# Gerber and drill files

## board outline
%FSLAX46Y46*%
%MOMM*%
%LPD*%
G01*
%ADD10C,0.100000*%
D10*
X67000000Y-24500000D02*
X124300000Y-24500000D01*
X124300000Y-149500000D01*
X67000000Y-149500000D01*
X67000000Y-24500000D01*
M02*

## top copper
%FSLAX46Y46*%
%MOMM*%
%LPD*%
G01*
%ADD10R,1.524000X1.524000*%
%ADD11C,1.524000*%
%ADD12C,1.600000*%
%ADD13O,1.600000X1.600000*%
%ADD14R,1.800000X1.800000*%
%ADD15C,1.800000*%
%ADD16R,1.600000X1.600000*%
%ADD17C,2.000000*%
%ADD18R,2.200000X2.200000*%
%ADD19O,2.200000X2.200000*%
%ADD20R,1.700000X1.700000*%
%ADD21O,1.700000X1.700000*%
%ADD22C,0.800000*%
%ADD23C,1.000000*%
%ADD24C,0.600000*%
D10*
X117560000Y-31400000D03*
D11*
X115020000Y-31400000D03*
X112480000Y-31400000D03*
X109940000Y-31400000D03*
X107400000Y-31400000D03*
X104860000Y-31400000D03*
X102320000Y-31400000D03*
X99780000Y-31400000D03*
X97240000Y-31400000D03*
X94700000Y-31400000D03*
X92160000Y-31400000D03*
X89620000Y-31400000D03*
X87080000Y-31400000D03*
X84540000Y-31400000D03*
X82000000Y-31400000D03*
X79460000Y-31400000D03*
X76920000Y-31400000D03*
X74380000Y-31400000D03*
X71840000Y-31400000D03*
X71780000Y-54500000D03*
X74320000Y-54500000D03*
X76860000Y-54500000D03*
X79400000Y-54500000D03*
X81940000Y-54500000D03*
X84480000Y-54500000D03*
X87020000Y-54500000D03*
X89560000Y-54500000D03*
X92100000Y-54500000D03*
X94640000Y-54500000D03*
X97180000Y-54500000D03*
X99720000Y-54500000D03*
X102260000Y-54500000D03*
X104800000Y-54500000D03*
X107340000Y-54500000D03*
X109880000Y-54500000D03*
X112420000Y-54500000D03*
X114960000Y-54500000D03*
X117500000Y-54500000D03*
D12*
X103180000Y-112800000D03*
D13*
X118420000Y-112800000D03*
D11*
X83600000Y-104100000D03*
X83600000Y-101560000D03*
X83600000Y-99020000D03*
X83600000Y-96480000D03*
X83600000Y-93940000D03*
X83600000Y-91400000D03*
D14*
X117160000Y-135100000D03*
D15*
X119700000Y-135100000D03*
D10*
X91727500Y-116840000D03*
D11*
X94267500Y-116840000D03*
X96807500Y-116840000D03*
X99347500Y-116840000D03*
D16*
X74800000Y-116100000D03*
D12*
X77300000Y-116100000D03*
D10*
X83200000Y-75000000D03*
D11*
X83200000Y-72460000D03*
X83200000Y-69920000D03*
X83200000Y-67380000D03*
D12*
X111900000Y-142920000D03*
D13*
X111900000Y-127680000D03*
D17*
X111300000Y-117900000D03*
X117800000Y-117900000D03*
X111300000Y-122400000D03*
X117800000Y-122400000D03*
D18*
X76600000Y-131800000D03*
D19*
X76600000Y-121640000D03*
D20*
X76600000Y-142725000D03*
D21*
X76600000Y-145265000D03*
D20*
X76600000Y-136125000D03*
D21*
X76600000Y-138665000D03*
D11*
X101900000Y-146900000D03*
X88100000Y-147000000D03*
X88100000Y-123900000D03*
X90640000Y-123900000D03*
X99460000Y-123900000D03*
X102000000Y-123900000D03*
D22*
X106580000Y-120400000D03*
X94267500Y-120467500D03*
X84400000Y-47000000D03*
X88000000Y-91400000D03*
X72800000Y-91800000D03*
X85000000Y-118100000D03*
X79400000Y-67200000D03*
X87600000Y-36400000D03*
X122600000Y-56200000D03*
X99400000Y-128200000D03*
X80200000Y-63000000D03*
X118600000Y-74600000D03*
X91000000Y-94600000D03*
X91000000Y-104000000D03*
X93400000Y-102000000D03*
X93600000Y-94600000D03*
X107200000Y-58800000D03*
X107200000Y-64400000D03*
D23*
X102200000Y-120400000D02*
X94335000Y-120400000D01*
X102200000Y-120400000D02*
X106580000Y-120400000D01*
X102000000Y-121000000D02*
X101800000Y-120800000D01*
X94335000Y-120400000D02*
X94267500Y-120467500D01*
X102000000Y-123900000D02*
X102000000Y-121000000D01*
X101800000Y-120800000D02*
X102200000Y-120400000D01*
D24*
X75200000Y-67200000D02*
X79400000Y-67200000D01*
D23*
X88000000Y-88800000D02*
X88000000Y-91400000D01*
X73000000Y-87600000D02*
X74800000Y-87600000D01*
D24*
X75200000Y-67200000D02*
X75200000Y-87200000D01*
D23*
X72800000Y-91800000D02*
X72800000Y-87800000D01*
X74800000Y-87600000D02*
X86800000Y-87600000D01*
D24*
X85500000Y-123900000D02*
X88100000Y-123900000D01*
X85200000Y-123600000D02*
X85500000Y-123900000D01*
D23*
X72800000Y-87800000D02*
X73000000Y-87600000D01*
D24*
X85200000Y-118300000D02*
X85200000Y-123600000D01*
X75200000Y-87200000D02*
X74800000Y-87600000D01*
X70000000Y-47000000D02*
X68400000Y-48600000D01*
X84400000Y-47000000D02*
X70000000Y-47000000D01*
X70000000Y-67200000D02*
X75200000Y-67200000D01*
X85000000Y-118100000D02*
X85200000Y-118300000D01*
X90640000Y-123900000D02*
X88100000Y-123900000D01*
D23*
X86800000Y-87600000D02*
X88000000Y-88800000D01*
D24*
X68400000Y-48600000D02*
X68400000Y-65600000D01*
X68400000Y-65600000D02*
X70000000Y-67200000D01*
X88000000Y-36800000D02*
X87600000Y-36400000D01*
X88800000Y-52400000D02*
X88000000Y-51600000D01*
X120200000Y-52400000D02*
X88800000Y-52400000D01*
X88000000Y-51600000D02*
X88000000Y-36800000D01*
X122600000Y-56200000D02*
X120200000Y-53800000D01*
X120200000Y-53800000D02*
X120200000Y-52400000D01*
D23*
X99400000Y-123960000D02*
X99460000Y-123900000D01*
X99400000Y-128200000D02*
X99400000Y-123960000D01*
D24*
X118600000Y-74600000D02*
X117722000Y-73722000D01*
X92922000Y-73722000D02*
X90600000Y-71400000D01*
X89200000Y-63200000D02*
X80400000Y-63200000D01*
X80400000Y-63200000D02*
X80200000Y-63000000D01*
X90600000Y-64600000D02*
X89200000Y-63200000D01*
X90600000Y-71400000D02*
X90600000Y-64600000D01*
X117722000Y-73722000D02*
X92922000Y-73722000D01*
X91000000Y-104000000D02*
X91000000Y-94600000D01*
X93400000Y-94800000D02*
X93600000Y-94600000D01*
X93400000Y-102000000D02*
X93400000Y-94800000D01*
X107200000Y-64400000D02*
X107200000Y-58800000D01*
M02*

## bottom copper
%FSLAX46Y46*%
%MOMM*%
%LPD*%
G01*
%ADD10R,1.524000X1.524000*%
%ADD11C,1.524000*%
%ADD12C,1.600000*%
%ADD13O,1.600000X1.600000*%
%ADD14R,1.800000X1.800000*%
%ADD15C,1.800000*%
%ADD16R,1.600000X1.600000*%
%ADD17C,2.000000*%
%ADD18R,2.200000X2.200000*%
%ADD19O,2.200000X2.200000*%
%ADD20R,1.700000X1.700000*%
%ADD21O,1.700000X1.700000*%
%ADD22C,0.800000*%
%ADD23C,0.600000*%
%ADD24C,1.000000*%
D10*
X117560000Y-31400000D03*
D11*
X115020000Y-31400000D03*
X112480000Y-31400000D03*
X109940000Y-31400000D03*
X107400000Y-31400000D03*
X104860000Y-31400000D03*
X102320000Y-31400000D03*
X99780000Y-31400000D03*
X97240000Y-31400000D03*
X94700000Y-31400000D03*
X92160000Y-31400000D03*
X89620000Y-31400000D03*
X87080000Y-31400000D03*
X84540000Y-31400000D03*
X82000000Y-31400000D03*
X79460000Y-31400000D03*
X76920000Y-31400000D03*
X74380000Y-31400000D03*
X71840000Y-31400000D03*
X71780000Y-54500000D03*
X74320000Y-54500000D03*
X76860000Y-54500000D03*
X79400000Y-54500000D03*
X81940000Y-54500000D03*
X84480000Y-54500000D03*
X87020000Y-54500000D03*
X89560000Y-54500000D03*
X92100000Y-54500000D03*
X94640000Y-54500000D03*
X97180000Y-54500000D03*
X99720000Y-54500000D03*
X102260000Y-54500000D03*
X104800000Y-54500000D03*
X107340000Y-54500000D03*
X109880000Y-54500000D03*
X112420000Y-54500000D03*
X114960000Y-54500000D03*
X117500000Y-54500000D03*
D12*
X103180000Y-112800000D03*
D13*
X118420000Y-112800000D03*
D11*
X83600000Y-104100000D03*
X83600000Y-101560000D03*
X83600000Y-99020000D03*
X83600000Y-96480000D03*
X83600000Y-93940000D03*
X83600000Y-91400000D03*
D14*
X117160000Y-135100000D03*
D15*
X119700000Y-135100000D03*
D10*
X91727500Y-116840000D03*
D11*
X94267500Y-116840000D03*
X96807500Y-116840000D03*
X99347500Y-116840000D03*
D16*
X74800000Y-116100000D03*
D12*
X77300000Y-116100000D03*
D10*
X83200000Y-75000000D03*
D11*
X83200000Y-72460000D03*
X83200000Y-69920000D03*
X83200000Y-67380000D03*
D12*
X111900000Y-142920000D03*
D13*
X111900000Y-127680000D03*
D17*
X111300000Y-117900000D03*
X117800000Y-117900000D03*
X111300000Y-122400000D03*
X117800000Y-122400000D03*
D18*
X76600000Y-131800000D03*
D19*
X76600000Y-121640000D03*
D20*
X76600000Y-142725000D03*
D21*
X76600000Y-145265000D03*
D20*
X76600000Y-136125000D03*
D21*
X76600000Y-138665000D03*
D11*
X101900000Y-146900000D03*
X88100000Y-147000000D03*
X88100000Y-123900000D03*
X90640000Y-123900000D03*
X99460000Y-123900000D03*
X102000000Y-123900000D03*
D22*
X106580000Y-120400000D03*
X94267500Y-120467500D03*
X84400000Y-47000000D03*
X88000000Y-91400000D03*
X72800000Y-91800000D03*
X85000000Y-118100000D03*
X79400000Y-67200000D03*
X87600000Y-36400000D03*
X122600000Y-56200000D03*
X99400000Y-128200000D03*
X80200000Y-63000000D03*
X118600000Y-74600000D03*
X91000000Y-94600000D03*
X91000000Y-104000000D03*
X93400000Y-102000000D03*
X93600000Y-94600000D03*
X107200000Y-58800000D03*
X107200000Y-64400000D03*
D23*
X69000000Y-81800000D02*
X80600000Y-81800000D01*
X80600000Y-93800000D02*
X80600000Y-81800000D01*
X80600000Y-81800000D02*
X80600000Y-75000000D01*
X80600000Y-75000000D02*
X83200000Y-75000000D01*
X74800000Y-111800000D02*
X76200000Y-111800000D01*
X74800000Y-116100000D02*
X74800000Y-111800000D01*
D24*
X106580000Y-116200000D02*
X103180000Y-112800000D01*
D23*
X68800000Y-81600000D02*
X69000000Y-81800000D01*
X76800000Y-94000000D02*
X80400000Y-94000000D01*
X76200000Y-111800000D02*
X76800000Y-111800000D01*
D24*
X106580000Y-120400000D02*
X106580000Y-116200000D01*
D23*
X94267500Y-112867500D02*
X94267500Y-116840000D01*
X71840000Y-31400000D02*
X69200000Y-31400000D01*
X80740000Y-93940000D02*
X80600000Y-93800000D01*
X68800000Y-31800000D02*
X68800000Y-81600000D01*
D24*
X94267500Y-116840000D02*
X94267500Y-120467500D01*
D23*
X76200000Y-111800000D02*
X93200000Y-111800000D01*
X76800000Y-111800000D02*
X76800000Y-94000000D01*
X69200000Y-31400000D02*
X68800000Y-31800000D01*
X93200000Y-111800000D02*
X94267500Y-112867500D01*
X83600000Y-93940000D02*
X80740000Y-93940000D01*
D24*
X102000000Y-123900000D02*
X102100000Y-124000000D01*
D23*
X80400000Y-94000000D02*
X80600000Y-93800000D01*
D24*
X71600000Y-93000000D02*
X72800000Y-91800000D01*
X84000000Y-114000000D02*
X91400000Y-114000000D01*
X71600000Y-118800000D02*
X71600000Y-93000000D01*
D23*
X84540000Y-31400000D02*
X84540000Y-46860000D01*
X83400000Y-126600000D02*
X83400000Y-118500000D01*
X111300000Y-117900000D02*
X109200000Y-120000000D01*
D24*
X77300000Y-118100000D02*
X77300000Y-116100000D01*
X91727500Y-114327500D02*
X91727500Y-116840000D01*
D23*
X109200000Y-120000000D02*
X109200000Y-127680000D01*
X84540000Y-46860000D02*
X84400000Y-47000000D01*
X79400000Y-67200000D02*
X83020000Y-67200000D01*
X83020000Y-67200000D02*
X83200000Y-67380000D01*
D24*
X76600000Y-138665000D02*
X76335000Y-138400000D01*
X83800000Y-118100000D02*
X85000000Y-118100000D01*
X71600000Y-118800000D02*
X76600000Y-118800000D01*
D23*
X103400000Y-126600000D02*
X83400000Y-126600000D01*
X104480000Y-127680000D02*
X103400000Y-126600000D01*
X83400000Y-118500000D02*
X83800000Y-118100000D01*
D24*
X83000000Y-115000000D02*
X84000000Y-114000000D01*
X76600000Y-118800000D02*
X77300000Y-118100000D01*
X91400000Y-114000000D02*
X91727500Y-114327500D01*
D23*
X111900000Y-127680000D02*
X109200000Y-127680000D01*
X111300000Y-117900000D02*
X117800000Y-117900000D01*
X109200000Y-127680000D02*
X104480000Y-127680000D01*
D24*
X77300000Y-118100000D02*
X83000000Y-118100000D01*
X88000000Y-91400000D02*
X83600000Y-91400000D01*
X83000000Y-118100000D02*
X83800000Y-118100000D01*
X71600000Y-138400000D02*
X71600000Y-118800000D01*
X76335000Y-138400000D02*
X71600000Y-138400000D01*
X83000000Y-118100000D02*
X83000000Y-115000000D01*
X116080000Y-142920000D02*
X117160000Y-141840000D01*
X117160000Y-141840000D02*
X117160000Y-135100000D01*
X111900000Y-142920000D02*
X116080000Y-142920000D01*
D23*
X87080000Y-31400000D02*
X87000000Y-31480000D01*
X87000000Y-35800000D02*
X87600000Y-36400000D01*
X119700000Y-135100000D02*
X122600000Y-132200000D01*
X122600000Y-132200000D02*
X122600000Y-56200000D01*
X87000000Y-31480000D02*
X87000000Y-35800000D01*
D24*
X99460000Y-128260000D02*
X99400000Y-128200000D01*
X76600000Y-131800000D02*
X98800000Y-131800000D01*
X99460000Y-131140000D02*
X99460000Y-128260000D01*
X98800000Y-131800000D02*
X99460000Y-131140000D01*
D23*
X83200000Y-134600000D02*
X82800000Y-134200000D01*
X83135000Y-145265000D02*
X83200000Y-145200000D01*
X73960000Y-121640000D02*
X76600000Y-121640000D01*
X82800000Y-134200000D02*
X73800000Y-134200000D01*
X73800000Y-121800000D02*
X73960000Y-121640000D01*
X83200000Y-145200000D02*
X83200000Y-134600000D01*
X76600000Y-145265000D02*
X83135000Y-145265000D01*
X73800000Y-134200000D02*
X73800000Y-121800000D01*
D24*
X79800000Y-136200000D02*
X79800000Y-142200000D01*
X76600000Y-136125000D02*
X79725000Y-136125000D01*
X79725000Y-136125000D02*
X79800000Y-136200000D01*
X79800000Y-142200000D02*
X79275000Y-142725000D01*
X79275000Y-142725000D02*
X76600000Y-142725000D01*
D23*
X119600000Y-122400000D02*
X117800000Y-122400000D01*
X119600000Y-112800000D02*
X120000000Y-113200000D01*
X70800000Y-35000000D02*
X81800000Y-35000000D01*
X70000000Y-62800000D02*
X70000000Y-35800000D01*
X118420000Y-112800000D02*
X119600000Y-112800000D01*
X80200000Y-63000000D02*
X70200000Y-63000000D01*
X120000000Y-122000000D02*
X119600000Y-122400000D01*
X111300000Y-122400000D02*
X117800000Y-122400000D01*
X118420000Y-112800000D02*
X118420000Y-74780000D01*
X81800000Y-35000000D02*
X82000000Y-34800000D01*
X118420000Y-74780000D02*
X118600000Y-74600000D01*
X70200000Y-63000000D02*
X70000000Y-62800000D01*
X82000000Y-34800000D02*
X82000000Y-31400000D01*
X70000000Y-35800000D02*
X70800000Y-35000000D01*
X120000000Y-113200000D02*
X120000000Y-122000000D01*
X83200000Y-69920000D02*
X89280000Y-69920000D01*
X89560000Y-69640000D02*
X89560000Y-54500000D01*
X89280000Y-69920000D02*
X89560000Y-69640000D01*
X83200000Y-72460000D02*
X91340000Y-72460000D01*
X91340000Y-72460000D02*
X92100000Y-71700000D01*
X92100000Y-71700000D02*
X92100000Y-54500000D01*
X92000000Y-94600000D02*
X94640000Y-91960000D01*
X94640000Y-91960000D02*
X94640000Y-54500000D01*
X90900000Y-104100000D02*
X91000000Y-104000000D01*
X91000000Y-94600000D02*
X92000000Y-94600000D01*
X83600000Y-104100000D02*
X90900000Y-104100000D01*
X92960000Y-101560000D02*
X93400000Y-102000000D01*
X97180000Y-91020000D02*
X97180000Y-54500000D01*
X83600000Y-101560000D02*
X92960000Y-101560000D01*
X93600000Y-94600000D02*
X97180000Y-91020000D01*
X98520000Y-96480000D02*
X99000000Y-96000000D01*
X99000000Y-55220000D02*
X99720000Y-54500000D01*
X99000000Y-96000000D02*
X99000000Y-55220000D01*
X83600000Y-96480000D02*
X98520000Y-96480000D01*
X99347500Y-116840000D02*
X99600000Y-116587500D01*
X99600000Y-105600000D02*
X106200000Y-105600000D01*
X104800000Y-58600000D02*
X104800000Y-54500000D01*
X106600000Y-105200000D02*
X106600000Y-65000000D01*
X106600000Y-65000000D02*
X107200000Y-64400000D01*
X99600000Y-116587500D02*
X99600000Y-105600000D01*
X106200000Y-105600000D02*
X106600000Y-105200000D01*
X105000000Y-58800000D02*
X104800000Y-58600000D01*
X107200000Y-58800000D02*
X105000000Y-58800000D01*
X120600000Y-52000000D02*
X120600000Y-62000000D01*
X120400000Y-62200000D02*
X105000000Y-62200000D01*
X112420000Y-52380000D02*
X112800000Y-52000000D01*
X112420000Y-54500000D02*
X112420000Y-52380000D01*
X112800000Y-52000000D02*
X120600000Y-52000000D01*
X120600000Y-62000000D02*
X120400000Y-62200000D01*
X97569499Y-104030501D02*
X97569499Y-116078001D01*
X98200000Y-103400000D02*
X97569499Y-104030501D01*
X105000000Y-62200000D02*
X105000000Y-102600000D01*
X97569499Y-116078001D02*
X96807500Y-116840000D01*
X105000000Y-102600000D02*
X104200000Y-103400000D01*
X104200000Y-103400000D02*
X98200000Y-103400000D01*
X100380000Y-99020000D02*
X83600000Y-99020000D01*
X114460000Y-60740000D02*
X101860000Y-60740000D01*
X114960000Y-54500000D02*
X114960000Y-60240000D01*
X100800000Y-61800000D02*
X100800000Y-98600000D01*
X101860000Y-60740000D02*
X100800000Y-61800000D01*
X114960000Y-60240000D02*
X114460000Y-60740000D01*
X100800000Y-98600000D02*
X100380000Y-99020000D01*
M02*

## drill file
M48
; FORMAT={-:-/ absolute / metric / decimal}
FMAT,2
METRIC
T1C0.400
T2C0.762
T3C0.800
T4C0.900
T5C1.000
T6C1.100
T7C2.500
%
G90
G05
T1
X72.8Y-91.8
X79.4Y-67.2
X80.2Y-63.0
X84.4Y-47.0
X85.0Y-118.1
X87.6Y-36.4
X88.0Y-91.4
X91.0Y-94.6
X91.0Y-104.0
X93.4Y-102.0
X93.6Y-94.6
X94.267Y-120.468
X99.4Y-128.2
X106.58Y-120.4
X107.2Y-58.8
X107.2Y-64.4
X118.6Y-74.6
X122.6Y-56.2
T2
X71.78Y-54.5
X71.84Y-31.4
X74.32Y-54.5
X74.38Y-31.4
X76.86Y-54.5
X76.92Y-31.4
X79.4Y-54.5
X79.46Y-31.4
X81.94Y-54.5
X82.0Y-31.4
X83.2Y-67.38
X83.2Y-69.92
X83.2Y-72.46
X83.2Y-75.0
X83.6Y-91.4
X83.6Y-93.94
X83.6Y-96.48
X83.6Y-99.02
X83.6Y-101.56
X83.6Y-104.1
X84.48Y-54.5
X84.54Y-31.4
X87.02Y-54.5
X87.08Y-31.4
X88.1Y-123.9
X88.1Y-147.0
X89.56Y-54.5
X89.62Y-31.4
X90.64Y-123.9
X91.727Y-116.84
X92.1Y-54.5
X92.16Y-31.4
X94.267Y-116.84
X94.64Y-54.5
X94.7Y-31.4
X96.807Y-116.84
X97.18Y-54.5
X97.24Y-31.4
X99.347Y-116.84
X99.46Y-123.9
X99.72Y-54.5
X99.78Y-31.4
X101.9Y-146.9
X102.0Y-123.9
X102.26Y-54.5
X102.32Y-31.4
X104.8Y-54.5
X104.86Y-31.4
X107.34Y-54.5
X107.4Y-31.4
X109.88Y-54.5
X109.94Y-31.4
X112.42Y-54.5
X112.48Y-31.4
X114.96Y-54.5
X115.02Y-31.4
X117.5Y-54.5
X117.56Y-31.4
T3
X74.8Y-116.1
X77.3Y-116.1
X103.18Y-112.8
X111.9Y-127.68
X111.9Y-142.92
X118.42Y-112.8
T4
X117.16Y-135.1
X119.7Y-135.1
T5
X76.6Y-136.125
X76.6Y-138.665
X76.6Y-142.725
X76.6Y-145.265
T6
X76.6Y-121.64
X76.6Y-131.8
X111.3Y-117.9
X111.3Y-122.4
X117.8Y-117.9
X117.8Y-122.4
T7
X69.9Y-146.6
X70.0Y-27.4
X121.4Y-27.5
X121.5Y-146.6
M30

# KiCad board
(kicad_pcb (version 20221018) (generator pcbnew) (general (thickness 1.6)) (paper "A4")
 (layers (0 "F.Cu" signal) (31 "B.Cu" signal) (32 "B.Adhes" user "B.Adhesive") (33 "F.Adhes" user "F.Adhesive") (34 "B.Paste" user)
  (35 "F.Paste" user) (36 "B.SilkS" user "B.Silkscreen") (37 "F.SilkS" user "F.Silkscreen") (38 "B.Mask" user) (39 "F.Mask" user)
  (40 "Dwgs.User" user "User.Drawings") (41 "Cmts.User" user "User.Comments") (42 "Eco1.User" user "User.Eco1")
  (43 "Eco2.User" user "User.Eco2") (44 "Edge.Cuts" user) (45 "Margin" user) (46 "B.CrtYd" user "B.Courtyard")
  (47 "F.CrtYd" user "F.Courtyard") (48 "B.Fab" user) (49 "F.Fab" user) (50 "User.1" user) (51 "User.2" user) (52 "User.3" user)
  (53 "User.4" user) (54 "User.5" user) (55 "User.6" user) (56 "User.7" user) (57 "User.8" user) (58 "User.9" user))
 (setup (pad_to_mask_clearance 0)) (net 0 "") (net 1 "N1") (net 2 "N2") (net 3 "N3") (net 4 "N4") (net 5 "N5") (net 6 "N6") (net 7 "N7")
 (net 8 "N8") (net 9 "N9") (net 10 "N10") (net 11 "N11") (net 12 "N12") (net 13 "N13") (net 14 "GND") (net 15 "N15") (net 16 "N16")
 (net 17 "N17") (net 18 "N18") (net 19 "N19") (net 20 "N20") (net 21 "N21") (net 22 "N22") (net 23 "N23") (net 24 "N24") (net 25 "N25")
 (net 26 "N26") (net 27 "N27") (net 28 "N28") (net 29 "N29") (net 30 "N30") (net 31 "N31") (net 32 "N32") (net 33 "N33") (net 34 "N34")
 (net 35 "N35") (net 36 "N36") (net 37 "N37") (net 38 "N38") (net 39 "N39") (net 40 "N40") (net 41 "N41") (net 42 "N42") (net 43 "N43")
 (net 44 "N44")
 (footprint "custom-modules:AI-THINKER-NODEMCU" (layer "F.Cu") (at 118.46 30.5 -90)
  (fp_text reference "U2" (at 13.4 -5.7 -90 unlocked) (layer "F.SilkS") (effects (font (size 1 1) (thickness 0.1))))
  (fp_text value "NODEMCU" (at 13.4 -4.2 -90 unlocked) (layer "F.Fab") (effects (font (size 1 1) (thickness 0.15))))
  (pad "1" thru_hole rect (at 0.9 0.9 270) (size 1.524 1.524) (drill 0.762) (layers "*.Cu" "*.Mask") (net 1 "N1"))
  (pad "2" thru_hole circle (at 0.9 3.44 270) (size 1.524 1.524) (drill 0.762) (layers "*.Cu" "*.Mask") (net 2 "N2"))
  (pad "3" thru_hole circle (at 0.9 5.98 270) (size 1.524 1.524) (drill 0.762) (layers "*.Cu" "*.Mask") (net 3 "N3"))
  (pad "4" thru_hole circle (at 0.9 8.52 270) (size 1.524 1.524) (drill 0.762) (layers "*.Cu" "*.Mask") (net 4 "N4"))
  (pad "5" thru_hole circle (at 0.9 11.06 270) (size 1.524 1.524) (drill 0.762) (layers "*.Cu" "*.Mask") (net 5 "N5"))
  (pad "6" thru_hole circle (at 0.9 13.6 270) (size 1.524 1.524) (drill 0.762) (layers "*.Cu" "*.Mask") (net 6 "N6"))
  (pad "7" thru_hole circle (at 0.9 16.14 270) (size 1.524 1.524) (drill 0.762) (layers "*.Cu" "*.Mask") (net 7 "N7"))
  (pad "8" thru_hole circle (at 0.9 18.68 270) (size 1.524 1.524) (drill 0.762) (layers "*.Cu" "*.Mask") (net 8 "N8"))
  (pad "9" thru_hole circle (at 0.9 21.22 270) (size 1.524 1.524) (drill 0.762) (layers "*.Cu" "*.Mask") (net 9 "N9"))
  (pad "10" thru_hole circle (at 0.9 23.76 270) (size 1.524 1.524) (drill 0.762) (layers "*.Cu" "*.Mask") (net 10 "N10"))
  (pad "11" thru_hole circle (at 0.9 26.3 270) (size 1.524 1.524) (drill 0.762) (layers "*.Cu" "*.Mask") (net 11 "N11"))
  (pad "12" thru_hole circle (at 0.9 28.84 270) (size 1.524 1.524) (drill 0.762) (layers "*.Cu" "*.Mask") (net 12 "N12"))
  (pad "13" thru_hole circle (at 0.9 31.38 270) (size 1.524 1.524) (drill 0.762) (layers "*.Cu" "*.Mask") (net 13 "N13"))
  (pad "14" thru_hole circle (at 0.9 33.92 270) (size 1.524 1.524) (drill 0.762) (layers "*.Cu" "*.Mask") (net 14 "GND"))
  (pad "15" thru_hole circle (at 0.9 36.46 270) (size 1.524 1.524) (drill 0.762) (layers "*.Cu" "*.Mask") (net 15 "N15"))
  (pad "16" thru_hole circle (at 0.9 39 270) (size 1.524 1.524) (drill 0.762) (layers "*.Cu" "*.Mask") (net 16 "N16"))
  (pad "17" thru_hole circle (at 0.9 41.54 270) (size 1.524 1.524) (drill 0.762) (layers "*.Cu" "*.Mask") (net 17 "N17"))
  (pad "18" thru_hole circle (at 0.9 44.08 270) (size 1.524 1.524) (drill 0.762) (layers "*.Cu" "*.Mask") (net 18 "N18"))
  (pad "19" thru_hole circle (at 0.9 46.62 270) (size 1.524 1.524) (drill 0.762) (layers "*.Cu" "*.Mask") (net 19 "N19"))
  (pad "20" thru_hole circle (at 24 46.68 270) (size 1.524 1.524) (drill 0.762) (layers "*.Cu" "*.Mask") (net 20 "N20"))
  (pad "21" thru_hole circle (at 24 44.14 270) (size 1.524 1.524) (drill 0.762) (layers "*.Cu" "*.Mask") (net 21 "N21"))
  (pad "22" thru_hole circle (at 24 41.6 270) (size 1.524 1.524) (drill 0.762) (layers "*.Cu" "*.Mask") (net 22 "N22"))
  (pad "23" thru_hole circle (at 24 39.06 270) (size 1.524 1.524) (drill 0.762) (layers "*.Cu" "*.Mask") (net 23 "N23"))
  (pad "24" thru_hole circle (at 24 36.52 270) (size 1.524 1.524) (drill 0.762) (layers "*.Cu" "*.Mask") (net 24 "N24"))
  (pad "25" thru_hole circle (at 24 33.98 270) (size 1.524 1.524) (drill 0.762) (layers "*.Cu" "*.Mask") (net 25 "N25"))
  (pad "26" thru_hole circle (at 24 31.44 270) (size 1.524 1.524) (drill 0.762) (layers "*.Cu" "*.Mask") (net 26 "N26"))
  (pad "27" thru_hole circle (at 24 28.9 270) (size 1.524 1.524) (drill 0.762) (layers "*.Cu" "*.Mask") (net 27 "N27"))
  (pad "28" thru_hole circle (at 24 26.36 270) (size 1.524 1.524) (drill 0.762) (layers "*.Cu" "*.Mask") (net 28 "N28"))
  (pad "29" thru_hole circle (at 24 23.82 270) (size 1.524 1.524) (drill 0.762) (layers "*.Cu" "*.Mask") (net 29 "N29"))
  (pad "30" thru_hole circle (at 24 21.28 270) (size 1.524 1.524) (drill 0.762) (layers "*.Cu" "*.Mask") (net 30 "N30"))
  (pad "31" thru_hole circle (at 24 18.74 270) (size 1.524 1.524) (drill 0.762) (layers "*.Cu" "*.Mask") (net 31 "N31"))
  (pad "32" thru_hole circle (at 24 16.2 270) (size 1.524 1.524) (drill 0.762) (layers "*.Cu" "*.Mask") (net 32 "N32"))
  (pad "33" thru_hole circle (at 24 13.66 270) (size 1.524 1.524) (drill 0.762) (layers "*.Cu" "*.Mask") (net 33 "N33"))
  (pad "34" thru_hole circle (at 24 11.12 270) (size 1.524 1.524) (drill 0.762) (layers "*.Cu" "*.Mask") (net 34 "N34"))
  (pad "35" thru_hole circle (at 24 8.58 270) (size 1.524 1.524) (drill 0.762) (layers "*.Cu" "*.Mask") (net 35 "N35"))
  (pad "36" thru_hole circle (at 24 6.04 270) (size 1.524 1.524) (drill 0.762) (layers "*.Cu" "*.Mask") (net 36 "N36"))
  (pad "37" thru_hole circle (at 24 3.5 270) (size 1.524 1.524) (drill 0.762) (layers "*.Cu" "*.Mask") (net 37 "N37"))
  (pad "38" thru_hole circle (at 24 0.96 270) (size 1.524 1.524) (drill 0.762) (layers "*.Cu" "*.Mask") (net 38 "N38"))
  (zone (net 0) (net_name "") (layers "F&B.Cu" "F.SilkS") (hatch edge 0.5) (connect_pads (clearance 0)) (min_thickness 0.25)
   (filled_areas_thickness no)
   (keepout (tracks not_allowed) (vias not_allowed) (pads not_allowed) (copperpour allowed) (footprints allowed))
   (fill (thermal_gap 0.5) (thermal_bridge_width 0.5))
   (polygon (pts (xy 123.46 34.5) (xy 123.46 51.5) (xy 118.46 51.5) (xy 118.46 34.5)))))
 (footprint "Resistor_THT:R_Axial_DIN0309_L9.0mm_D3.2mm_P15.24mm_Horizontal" (layer "F.Cu") (at 103.18 112.8)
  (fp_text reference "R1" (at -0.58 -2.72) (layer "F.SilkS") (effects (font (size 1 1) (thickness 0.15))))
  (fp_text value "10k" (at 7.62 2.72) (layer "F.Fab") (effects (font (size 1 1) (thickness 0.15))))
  (pad "1" thru_hole circle (at 0 0) (size 1.6 1.6) (drill 0.8) (layers "*.Cu" "*.Mask") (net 19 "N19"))
  (pad "2" thru_hole oval (at 15.24 0) (size 1.6 1.6) (drill 0.8) (layers "*.Cu" "*.Mask") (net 15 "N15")))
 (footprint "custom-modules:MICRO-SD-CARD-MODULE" (layer "F.Cu") (at 82.5 110.1 90)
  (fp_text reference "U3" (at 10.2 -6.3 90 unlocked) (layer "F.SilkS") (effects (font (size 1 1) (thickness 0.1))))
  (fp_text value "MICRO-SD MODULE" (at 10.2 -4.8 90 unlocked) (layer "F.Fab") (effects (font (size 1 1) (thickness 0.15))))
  (pad "1" thru_hole circle (at 6 1.1 90) (size 1.524 1.524) (drill 0.762) (layers "*.Cu" "*.Mask") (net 29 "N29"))
  (pad "2" thru_hole circle (at 8.54 1.1 90) (size 1.524 1.524) (drill 0.762) (layers "*.Cu" "*.Mask") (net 30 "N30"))
  (pad "3" thru_hole circle (at 11.08 1.1 90) (size 1.524 1.524) (drill 0.762) (layers "*.Cu" "*.Mask") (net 37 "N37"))
  (pad "4" thru_hole circle (at 13.62 1.1 90) (size 1.524 1.524) (drill 0.762) (layers "*.Cu" "*.Mask") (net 31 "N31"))
  (pad "5" thru_hole circle (at 16.16 1.1 90) (size 1.524 1.524) (drill 0.762) (layers "*.Cu" "*.Mask") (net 19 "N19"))
  (pad "6" thru_hole circle (at 18.7 1.1 90) (size 1.524 1.524) (drill 0.762) (layers "*.Cu" "*.Mask") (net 14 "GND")))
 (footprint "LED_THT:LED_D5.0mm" (layer "F.Cu") (at 117.16 135.1)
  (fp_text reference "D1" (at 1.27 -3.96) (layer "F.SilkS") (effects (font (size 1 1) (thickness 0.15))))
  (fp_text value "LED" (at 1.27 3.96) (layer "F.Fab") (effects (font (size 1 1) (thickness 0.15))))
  (pad "1" thru_hole rect (at 0 0) (size 1.8 1.8) (drill 0.9) (layers "*.Cu" "*.Mask") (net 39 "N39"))
  (pad "2" thru_hole circle (at 2.54 0) (size 1.8 1.8) (drill 0.9) (layers "*.Cu" "*.Mask") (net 13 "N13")))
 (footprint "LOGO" (layer "F.Cu") (at 75 91.4 90)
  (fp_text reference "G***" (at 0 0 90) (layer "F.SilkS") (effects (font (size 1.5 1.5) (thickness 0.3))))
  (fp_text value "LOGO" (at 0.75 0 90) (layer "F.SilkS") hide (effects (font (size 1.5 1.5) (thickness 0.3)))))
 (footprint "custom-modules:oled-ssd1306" (layer "F.Cu") (at 81.0595 115.443)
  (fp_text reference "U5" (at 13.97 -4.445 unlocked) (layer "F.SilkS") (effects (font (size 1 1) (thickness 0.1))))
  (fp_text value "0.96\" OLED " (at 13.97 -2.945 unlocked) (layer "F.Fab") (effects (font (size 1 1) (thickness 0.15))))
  (pad "1" thru_hole rect (at 10.668 1.397) (size 1.524 1.524) (drill 0.762) (layers "*.Cu" "*.Mask") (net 14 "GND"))
  (pad "2" thru_hole circle (at 13.208 1.397) (size 1.524 1.524) (drill 0.762) (layers "*.Cu" "*.Mask") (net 19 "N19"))
  (pad "3" thru_hole circle (at 15.748 1.397) (size 1.524 1.524) (drill 0.762) (layers "*.Cu" "*.Mask") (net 36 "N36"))
  (pad "4" thru_hole circle (at 18.288 1.397) (size 1.524 1.524) (drill 0.762) (layers "*.Cu" "*.Mask") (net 33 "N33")))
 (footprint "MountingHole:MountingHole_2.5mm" (layer "F.Cu") (at 69.9 146.6)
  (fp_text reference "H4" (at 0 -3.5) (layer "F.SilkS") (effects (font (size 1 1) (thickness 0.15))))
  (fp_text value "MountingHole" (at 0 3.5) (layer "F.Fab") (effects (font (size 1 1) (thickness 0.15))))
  (pad "" np_thru_hole circle (at 0 0) (size 2.5 2.5) (drill 2.5) (layers "*.Cu" "*.Mask")))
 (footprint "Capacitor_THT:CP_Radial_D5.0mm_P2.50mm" (layer "F.Cu") (at 74.8 116.1)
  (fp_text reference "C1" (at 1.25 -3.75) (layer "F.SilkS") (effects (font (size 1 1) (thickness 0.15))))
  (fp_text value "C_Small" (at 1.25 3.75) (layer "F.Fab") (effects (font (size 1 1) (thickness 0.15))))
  (pad "1" thru_hole rect (at 0 0) (size 1.6 1.6) (drill 0.8) (layers "*.Cu" "*.Mask") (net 19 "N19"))
  (pad "2" thru_hole circle (at 2.5 0) (size 1.6 1.6) (drill 0.8) (layers "*.Cu" "*.Mask") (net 14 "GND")))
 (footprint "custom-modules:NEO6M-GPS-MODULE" (layer "F.Cu") (at 82.2 84.3 90)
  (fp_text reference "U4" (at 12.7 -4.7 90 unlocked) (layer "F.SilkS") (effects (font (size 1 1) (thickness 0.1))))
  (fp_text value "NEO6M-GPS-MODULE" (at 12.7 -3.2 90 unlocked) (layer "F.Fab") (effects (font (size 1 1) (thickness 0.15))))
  (pad "1" thru_hole rect (at 9.3 1 90) (size 1.524 1.524) (drill 0.762) (layers "*.Cu" "*.Mask") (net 19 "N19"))
  (pad "2" thru_hole circle (at 11.84 1 90) (size 1.524 1.524) (drill 0.762) (layers "*.Cu" "*.Mask") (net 28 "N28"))
  (pad "3" thru_hole circle (at 14.38 1 90) (size 1.524 1.524) (drill 0.762) (layers "*.Cu" "*.Mask") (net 27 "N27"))
  (pad "4" thru_hole circle (at 16.92 1 90) (size 1.524 1.524) (drill 0.762) (layers "*.Cu" "*.Mask") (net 14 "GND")))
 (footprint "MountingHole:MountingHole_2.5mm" (layer "F.Cu") (at 121.4 27.5)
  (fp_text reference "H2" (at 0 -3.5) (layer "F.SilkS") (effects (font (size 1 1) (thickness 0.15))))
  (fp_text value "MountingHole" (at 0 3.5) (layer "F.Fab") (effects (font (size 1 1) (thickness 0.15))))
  (pad "" np_thru_hole circle (at 0 0) (size 2.5 2.5) (drill 2.5) (layers "*.Cu" "*.Mask")))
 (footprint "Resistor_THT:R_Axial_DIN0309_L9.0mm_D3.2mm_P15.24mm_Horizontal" (layer "F.Cu") (at 111.9 142.92 90)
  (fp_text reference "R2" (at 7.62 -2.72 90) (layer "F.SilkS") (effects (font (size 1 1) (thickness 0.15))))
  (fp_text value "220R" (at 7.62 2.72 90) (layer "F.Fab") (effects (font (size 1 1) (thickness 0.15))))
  (pad "1" thru_hole circle (at 0 0 90) (size 1.6 1.6) (drill 0.8) (layers "*.Cu" "*.Mask") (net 39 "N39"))
  (pad "2" thru_hole oval (at 15.24 0 90) (size 1.6 1.6) (drill 0.8) (layers "*.Cu" "*.Mask") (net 14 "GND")))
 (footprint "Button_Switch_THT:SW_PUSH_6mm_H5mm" (layer "F.Cu") (at 111.3 117.9)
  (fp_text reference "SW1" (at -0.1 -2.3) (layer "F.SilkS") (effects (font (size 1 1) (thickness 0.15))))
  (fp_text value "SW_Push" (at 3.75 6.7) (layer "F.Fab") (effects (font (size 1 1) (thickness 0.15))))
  (pad "1" thru_hole circle (at 0 0 90) (size 2 2) (drill 1.1) (layers "*.Cu" "*.Mask") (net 14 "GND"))
  (pad "1" thru_hole circle (at 6.5 0 90) (size 2 2) (drill 1.1) (layers "*.Cu" "*.Mask") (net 14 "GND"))
  (pad "2" thru_hole circle (at 0 4.5 90) (size 2 2) (drill 1.1) (layers "*.Cu" "*.Mask") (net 15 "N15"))
  (pad "2" thru_hole circle (at 6.5 4.5 90) (size 2 2) (drill 1.1) (layers "*.Cu" "*.Mask") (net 15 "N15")))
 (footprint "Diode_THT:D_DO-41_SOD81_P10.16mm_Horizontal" (layer "F.Cu") (at 76.6 131.8 90)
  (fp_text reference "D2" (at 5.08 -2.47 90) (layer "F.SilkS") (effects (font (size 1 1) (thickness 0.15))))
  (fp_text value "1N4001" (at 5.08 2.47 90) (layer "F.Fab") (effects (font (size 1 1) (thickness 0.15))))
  (pad "1" thru_hole rect (at 0 0 90) (size 2.2 2.2) (drill 1.1) (layers "*.Cu" "*.Mask") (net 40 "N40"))
  (pad "2" thru_hole oval (at 10.16 0 90) (size 2.2 2.2) (drill 1.1) (layers "*.Cu" "*.Mask") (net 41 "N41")))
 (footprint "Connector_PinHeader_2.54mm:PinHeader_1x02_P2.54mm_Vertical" (layer "F.Cu") (at 76.6 142.725)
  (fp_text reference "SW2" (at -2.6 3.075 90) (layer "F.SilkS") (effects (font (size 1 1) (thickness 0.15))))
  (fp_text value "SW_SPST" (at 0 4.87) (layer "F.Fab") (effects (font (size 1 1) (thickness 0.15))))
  (pad "1" thru_hole rect (at 0 0) (size 1.7 1.7) (drill 1) (layers "*.Cu" "*.Mask") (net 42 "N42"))
  (pad "2" thru_hole oval (at 0 2.54) (size 1.7 1.7) (drill 1) (layers "*.Cu" "*.Mask") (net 41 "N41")))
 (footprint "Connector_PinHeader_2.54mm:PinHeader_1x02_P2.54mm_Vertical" (layer "F.Cu") (at 76.6 136.125)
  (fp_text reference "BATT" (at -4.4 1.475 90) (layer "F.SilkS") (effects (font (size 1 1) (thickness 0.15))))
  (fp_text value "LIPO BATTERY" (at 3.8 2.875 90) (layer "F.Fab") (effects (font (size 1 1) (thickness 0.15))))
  (pad "1" thru_hole rect (at 0 0) (size 1.7 1.7) (drill 1) (layers "*.Cu" "*.Mask") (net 42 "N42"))
  (pad "2" thru_hole oval (at 0 2.54) (size 1.7 1.7) (drill 1) (layers "*.Cu" "*.Mask") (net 14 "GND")))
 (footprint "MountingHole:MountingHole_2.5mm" (layer "F.Cu") (at 70 27.4)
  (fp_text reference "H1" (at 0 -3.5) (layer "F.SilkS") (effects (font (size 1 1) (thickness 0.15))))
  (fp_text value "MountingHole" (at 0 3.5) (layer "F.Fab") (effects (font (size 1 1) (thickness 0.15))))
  (pad "" np_thru_hole circle (at 0 0) (size 2.5 2.5) (drill 2.5) (layers "*.Cu" "*.Mask")))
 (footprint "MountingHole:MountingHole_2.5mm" (layer "F.Cu") (at 121.5 146.6)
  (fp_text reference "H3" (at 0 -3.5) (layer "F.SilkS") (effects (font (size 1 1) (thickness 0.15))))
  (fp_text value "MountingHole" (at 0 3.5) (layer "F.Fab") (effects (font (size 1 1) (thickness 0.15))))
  (pad "" np_thru_hole circle (at 0 0) (size 2.5 2.5) (drill 2.5) (layers "*.Cu" "*.Mask")))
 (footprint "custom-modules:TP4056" (layer "B.Cu") (at 103.7 149.4 90)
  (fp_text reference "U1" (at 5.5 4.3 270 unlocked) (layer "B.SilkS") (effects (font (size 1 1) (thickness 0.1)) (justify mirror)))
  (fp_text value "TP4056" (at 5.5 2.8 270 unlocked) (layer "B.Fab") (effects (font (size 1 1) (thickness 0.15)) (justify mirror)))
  (pad "1" thru_hole circle (at 2.5 -1.8 90) (size 1.524 1.524) (drill 0.762) (layers "*.Cu" "*.Mask") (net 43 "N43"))
  (pad "2" thru_hole circle (at 2.4 -15.6 90) (size 1.524 1.524) (drill 0.762) (layers "*.Cu" "*.Mask") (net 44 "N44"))
  (pad "3" thru_hole circle (at 25.5 -15.6 90) (size 1.524 1.524) (drill 0.762) (layers "*.Cu" "*.Mask") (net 14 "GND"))
  (pad "4" thru_hole circle (at 25.5 -13.06 90) (size 1.524 1.524) (drill 0.762) (layers "*.Cu" "*.Mask") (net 14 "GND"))
  (pad "5" thru_hole circle (at 25.5 -4.24 90) (size 1.524 1.524) (drill 0.762) (layers "*.Cu" "*.Mask") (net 40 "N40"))
  (pad "6" thru_hole circle (at 25.5 -1.7 90) (size 1.524 1.524) (drill 0.762) (layers "*.Cu" "*.Mask") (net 19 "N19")))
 (gr_rect (start 67 24.5) (end 124.3 149.5) (stroke (width 0.1) (type default)) (fill none) (layer "Edge.Cuts"))
 (segment (start 102.2 120.4) (end 94.335 120.4) (width 1) (layer "F.Cu") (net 19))
 (segment (start 102.2 120.4) (end 106.58 120.4) (width 1) (layer "F.Cu") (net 19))
 (segment (start 102 121) (end 101.8 120.8) (width 1) (layer "F.Cu") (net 19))
 (segment (start 94.335 120.4) (end 94.2675 120.4675) (width 1) (layer "F.Cu") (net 19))
 (segment (start 102 123.9) (end 102 121) (width 1) (layer "F.Cu") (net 19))
 (segment (start 101.8 120.8) (end 102.2 120.4) (width 1) (layer "F.Cu") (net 19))
 (via (at 106.58 120.4) (size 0.8) (drill 0.4) (layers "F.Cu" "B.Cu") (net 19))
 (via (at 94.2675 120.4675) (size 0.8) (drill 0.4) (layers "F.Cu" "B.Cu") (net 19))
 (segment (start 69 81.8) (end 80.6 81.8) (width 0.6) (layer "B.Cu") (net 19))
 (segment (start 80.6 93.8) (end 80.6 81.8) (width 0.6) (layer "B.Cu") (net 19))
 (segment (start 80.6 81.8) (end 80.6 75) (width 0.6) (layer "B.Cu") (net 19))
 (segment (start 80.6 75) (end 83.2 75) (width 0.6) (layer "B.Cu") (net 19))
 (segment (start 74.8 111.8) (end 76.2 111.8) (width 0.6) (layer "B.Cu") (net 19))
 (segment (start 74.8 116.1) (end 74.8 111.8) (width 0.6) (layer "B.Cu") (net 19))
 (segment (start 106.58 116.2) (end 103.18 112.8) (width 1) (layer "B.Cu") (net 19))
 (segment (start 68.8 81.6) (end 69 81.8) (width 0.6) (layer "B.Cu") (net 19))
 (segment (start 76.8 94) (end 80.4 94) (width 0.6) (layer "B.Cu") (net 19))
 (segment (start 76.2 111.8) (end 76.8 111.8) (width 0.6) (layer "B.Cu") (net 19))
 (segment (start 106.58 120.4) (end 106.58 116.2) (width 1) (layer "B.Cu") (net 19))
 (segment (start 94.2675 112.8675) (end 94.2675 116.84) (width 0.6) (layer "B.Cu") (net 19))
 (segment (start 71.84 31.4) (end 69.2 31.4) (width 0.6) (layer "B.Cu") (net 19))
 (segment (start 80.74 93.94) (end 80.6 93.8) (width 0.6) (layer "B.Cu") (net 19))
 (segment (start 68.8 31.8) (end 68.8 81.6) (width 0.6) (layer "B.Cu") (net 19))
 (segment (start 94.2675 116.84) (end 94.2675 120.4675) (width 1) (layer "B.Cu") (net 19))
 (segment (start 76.2 111.8) (end 93.2 111.8) (width 0.6) (layer "B.Cu") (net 19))
 (segment (start 76.8 111.8) (end 76.8 94) (width 0.6) (layer "B.Cu") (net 19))
 (segment (start 69.2 31.4) (end 68.8 31.8) (width 0.6) (layer "B.Cu") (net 19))
 (segment (start 93.2 111.8) (end 94.2675 112.8675) (width 0.6) (layer "B.Cu") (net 19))
 (segment (start 83.6 93.94) (end 80.74 93.94) (width 0.6) (layer "B.Cu") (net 19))
 (segment (start 102 123.9) (end 102.1 124) (width 1) (layer "B.Cu") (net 19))
 (segment (start 80.4 94) (end 80.6 93.8) (width 0.6) (layer "B.Cu") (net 19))
 (segment (start 75.2 67.2) (end 79.4 67.2) (width 0.6) (layer "F.Cu") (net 14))
 (segment (start 88 88.8) (end 88 91.4) (width 1) (layer "F.Cu") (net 14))
 (segment (start 73 87.6) (end 74.8 87.6) (width 1) (layer "F.Cu") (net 14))
 (segment (start 75.2 67.2) (end 75.2 87.2) (width 0.6) (layer "F.Cu") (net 14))
 (segment (start 72.8 91.8) (end 72.8 87.8) (width 1) (layer "F.Cu") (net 14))
 (segment (start 74.8 87.6) (end 86.8 87.6) (width 1) (layer "F.Cu") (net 14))
 (segment (start 85.5 123.9) (end 88.1 123.9) (width 0.6) (layer "F.Cu") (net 14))
 (segment (start 85.2 123.6) (end 85.5 123.9) (width 0.6) (layer "F.Cu") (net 14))
 (segment (start 72.8 87.8) (end 73 87.6) (width 1) (layer "F.Cu") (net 14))
 (segment (start 85.2 118.3) (end 85.2 123.6) (width 0.6) (layer "F.Cu") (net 14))
 (segment (start 75.2 87.2) (end 74.8 87.6) (width 0.6) (layer "F.Cu") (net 14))
 (segment (start 70 47) (end 68.4 48.6) (width 0.6) (layer "F.Cu") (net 14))
 (segment (start 84.4 47) (end 70 47) (width 0.6) (layer "F.Cu") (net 14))
 (segment (start 70 67.2) (end 75.2 67.2) (width 0.6) (layer "F.Cu") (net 14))
 (segment (start 85 118.1) (end 85.2 118.3) (width 0.6) (layer "F.Cu") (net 14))
 (segment (start 90.64 123.9) (end 88.1 123.9) (width 0.6) (layer "F.Cu") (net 14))
 (segment (start 86.8 87.6) (end 88 88.8) (width 1) (layer "F.Cu") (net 14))
 (segment (start 68.4 48.6) (end 68.4 65.6) (width 0.6) (layer "F.Cu") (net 14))
 (segment (start 68.4 65.6) (end 70 67.2) (width 0.6) (layer "F.Cu") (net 14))
 (via (at 84.4 47) (size 0.8) (drill 0.4) (layers "F.Cu" "B.Cu") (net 14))
 (via (at 88 91.4) (size 0.8) (drill 0.4) (layers "F.Cu" "B.Cu") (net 14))
 (via (at 72.8 91.8) (size 0.8) (drill 0.4) (layers "F.Cu" "B.Cu") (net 14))
 (via (at 85 118.1) (size 0.8) (drill 0.4) (layers "F.Cu" "B.Cu") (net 14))
 (via (at 79.4 67.2) (size 0.8) (drill 0.4) (layers "F.Cu" "B.Cu") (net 14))
 (segment (start 71.6 93) (end 72.8 91.8) (width 1) (layer "B.Cu") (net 14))
 (segment (start 84 114) (end 91.4 114) (width 1) (layer "B.Cu") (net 14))
 (segment (start 71.6 118.8) (end 71.6 93) (width 1) (layer "B.Cu") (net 14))
 (segment (start 84.54 31.4) (end 84.54 46.86) (width 0.6) (layer "B.Cu") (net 14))
 (segment (start 83.4 126.6) (end 83.4 118.5) (width 0.6) (layer "B.Cu") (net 14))
 (segment (start 111.3 117.9) (end 109.2 120) (width 0.6) (layer "B.Cu") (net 14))
 (segment (start 77.3 118.1) (end 77.3 116.1) (width 1) (layer "B.Cu") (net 14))
 (segment (start 91.7275 114.3275) (end 91.7275 116.84) (width 1) (layer "B.Cu") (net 14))
 (segment (start 109.2 120) (end 109.2 127.68) (width 0.6) (layer "B.Cu") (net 14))
 (segment (start 84.54 46.86) (end 84.4 47) (width 0.6) (layer "B.Cu") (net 14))
 (segment (start 79.4 67.2) (end 83.02 67.2) (width 0.6) (layer "B.Cu") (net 14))
 (segment (start 83.02 67.2) (end 83.2 67.38) (width 0.6) (layer "B.Cu") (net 14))
 (segment (start 76.6 138.665) (end 76.335 138.4) (width 1) (layer "B.Cu") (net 14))
 (segment (start 83.8 118.1) (end 85 118.1) (width 1) (layer "B.Cu") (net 14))
 (segment (start 71.6 118.8) (end 76.6 118.8) (width 1) (layer "B.Cu") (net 14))
 (segment (start 103.4 126.6) (end 83.4 126.6) (width 0.6) (layer "B.Cu") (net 14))
 (segment (start 104.48 127.68) (end 103.4 126.6) (width 0.6) (layer "B.Cu") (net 14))
 (segment (start 83.4 118.5) (end 83.8 118.1) (width 0.6) (layer "B.Cu") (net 14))
 (segment (start 83 115) (end 84 114) (width 1) (layer "B.Cu") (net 14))
 (segment (start 76.6 118.8) (end 77.3 118.1) (width 1) (layer "B.Cu") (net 14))
 (segment (start 91.4 114) (end 91.7275 114.3275) (width 1) (layer "B.Cu") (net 14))
 (segment (start 111.9 127.68) (end 109.2 127.68) (width 0.6) (layer "B.Cu") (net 14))
 (segment (start 111.3 117.9) (end 117.8 117.9) (width 0.6) (layer "B.Cu") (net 14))
 (segment (start 109.2 127.68) (end 104.48 127.68) (width 0.6) (layer "B.Cu") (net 14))
 (segment (start 77.3 118.1) (end 83 118.1) (width 1) (layer "B.Cu") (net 14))
 (segment (start 88 91.4) (end 83.6 91.4) (width 1) (layer "B.Cu") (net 14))
 (segment (start 83 118.1) (end 83.8 118.1) (width 1) (layer "B.Cu") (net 14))
 (segment (start 71.6 138.4) (end 71.6 118.8) (width 1) (layer "B.Cu") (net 14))
 (segment (start 76.335 138.4) (end 71.6 138.4) (width 1) (layer "B.Cu") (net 14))
 (segment (start 83 118.1) (end 83 115) (width 1) (layer "B.Cu") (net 14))
 (segment (start 116.08 142.92) (end 117.16 141.84) (width 1) (layer "B.Cu") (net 39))
 (segment (start 117.16 141.84) (end 117.16 135.1) (width 1) (layer "B.Cu") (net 39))
 (segment (start 111.9 142.92) (end 116.08 142.92) (width 1) (layer "B.Cu") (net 39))
 (segment (start 88 36.8) (end 87.6 36.4) (width 0.6) (layer "F.Cu") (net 13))
 (segment (start 88.8 52.4) (end 88 51.6) (width 0.6) (layer "F.Cu") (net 13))
 (segment (start 120.2 52.4) (end 88.8 52.4) (width 0.6) (layer "F.Cu") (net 13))
 (segment (start 88 51.6) (end 88 36.8) (width 0.6) (layer "F.Cu") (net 13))
 (segment (start 122.6 56.2) (end 120.2 53.8) (width 0.6) (layer "F.Cu") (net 13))
 (segment (start 120.2 53.8) (end 120.2 52.4) (width 0.6) (layer "F.Cu") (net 13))
 (via (at 87.6 36.4) (size 0.8) (drill 0.4) (layers "F.Cu" "B.Cu") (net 13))
 (via (at 122.6 56.2) (size 0.8) (drill 0.4) (layers "F.Cu" "B.Cu") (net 13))
 (segment (start 87.08 31.4) (end 87 31.48) (width 0.6) (layer "B.Cu") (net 13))
 (segment (start 87 35.8) (end 87.6 36.4) (width 0.6) (layer "B.Cu") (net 13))
 (segment (start 119.7 135.1) (end 122.6 132.2) (width 0.6) (layer "B.Cu") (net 13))
 (segment (start 122.6 132.2) (end 122.6 56.2) (width 0.6) (layer "B.Cu") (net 13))
 (segment (start 87 31.48) (end 87 35.8) (width 0.6) (layer "B.Cu") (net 13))
 (segment (start 99.4 123.96) (end 99.46 123.9) (width 1) (layer "F.Cu") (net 40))
 (segment (start 99.4 128.2) (end 99.4 123.96) (width 1) (layer "F.Cu") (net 40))
 (via (at 99.4 128.2) (size 0.8) (drill 0.4) (layers "F.Cu" "B.Cu") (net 40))
 (segment (start 99.46 128.26) (end 99.4 128.2) (width 1) (layer "B.Cu") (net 40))
 (segment (start 76.6 131.8) (end 98.8 131.8) (width 1) (layer "B.Cu") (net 40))
 (segment (start 99.46 131.14) (end 99.46 128.26) (width 1) (layer "B.Cu") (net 40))
 (segment (start 98.8 131.8) (end 99.46 131.14) (width 1) (layer "B.Cu") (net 40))
 (segment (start 83.2 134.6) (end 82.8 134.2) (width 0.6) (layer "B.Cu") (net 41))
 (segment (start 83.135 145.265) (end 83.2 145.2) (width 0.6) (layer "B.Cu") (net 41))
 (segment (start 73.96 121.64) (end 76.6 121.64) (width 0.6) (layer "B.Cu") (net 41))
 (segment (start 82.8 134.2) (end 73.8 134.2) (width 0.6) (layer "B.Cu") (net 41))
 (segment (start 73.8 121.8) (end 73.96 121.64) (width 0.6) (layer "B.Cu") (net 41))
 (segment (start 83.2 145.2) (end 83.2 134.6) (width 0.6) (layer "B.Cu") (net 41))
 (segment (start 76.6 145.265) (end 83.135 145.265) (width 0.6) (layer "B.Cu") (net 41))
 (segment (start 73.8 134.2) (end 73.8 121.8) (width 0.6) (layer "B.Cu") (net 41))
 (segment (start 79.8 136.2) (end 79.8 142.2) (width 1) (layer "B.Cu") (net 42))
 (segment (start 76.6 136.125) (end 79.725 136.125) (width 1) (layer "B.Cu") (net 42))
 (segment (start 79.725 136.125) (end 79.8 136.2) (width 1) (layer "B.Cu") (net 42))
 (segment (start 79.8 142.2) (end 79.275 142.725) (width 1) (layer "B.Cu") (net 42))
 (segment (start 79.275 142.725) (end 76.6 142.725) (width 1) (layer "B.Cu") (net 42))
 (segment (start 118.6 74.6) (end 117.722 73.722) (width 0.6) (layer "F.Cu") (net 15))
 (segment (start 92.922 73.722) (end 90.6 71.4) (width 0.6) (layer "F.Cu") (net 15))
 (segment (start 89.2 63.2) (end 80.4 63.2) (width 0.6) (layer "F.Cu") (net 15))
 (segment (start 80.4 63.2) (end 80.2 63) (width 0.6) (layer "F.Cu") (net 15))
 (segment (start 90.6 64.6) (end 89.2 63.2) (width 0.6) (layer "F.Cu") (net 15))
 (segment (start 90.6 71.4) (end 90.6 64.6) (width 0.6) (layer "F.Cu") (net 15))
 (segment (start 117.722 73.722) (end 92.922 73.722) (width 0.6) (layer "F.Cu") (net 15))
 (via (at 80.2 63) (size 0.8) (drill 0.4) (layers "F.Cu" "B.Cu") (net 15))
 (via (at 118.6 74.6) (size 0.8) (drill 0.4) (layers "F.Cu" "B.Cu") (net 15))
 (segment (start 119.6 122.4) (end 117.8 122.4) (width 0.6) (layer "B.Cu") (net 15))
 (segment (start 119.6 112.8) (end 120 113.2) (width 0.6) (layer "B.Cu") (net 15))
 (segment (start 70.8 35) (end 81.8 35) (width 0.6) (layer "B.Cu") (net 15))
 (segment (start 70 62.8) (end 70 35.8) (width 0.6) (layer "B.Cu") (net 15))
 (segment (start 118.42 112.8) (end 119.6 112.8) (width 0.6) (layer "B.Cu") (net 15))
 (segment (start 80.2 63) (end 70.2 63) (width 0.6) (layer "B.Cu") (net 15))
 (segment (start 120 122) (end 119.6 122.4) (width 0.6) (layer "B.Cu") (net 15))
 (segment (start 111.3 122.4) (end 117.8 122.4) (width 0.6) (layer "B.Cu") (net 15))
 (segment (start 118.42 112.8) (end 118.42 74.78) (width 0.6) (layer "B.Cu") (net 15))
 (segment (start 81.8 35) (end 82 34.8) (width 0.6) (layer "B.Cu") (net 15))
 (segment (start 118.42 74.78) (end 118.6 74.6) (width 0.6) (layer "B.Cu") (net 15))
 (segment (start 70.2 63) (end 70 62.8) (width 0.6) (layer "B.Cu") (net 15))
 (segment (start 82 34.8) (end 82 31.4) (width 0.6) (layer "B.Cu") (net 15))
 (segment (start 70 35.8) (end 70.8 35) (width 0.6) (layer "B.Cu") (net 15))
 (segment (start 120 113.2) (end 120 122) (width 0.6) (layer "B.Cu") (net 15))
 (segment (start 83.2 69.92) (end 89.28 69.92) (width 0.6) (layer "B.Cu") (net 27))
 (segment (start 89.56 69.64) (end 89.56 54.5) (width 0.6) (layer "B.Cu") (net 27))
 (segment (start 89.28 69.92) (end 89.56 69.64) (width 0.6) (layer "B.Cu") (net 27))
 (segment (start 83.2 72.46) (end 91.34 72.46) (width 0.6) (layer "B.Cu") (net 28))
 (segment (start 91.34 72.46) (end 92.1 71.7) (width 0.6) (layer "B.Cu") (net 28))
 (segment (start 92.1 71.7) (end 92.1 54.5) (width 0.6) (layer "B.Cu") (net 28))
 (segment (start 91 104) (end 91 94.6) (width 0.6) (layer "F.Cu") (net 29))
 (via (at 91 94.6) (size 0.8) (drill 0.4) (layers "F.Cu" "B.Cu") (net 29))
 (via (at 91 104) (size 0.8) (drill 0.4) (layers "F.Cu" "B.Cu") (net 29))
 (segment (start 92 94.6) (end 94.64 91.96) (width 0.6) (layer "B.Cu") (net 29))
 (segment (start 94.64 91.96) (end 94.64 54.5) (width 0.6) (layer "B.Cu") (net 29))
 (segment (start 90.9 104.1) (end 91 104) (width 0.6) (layer "B.Cu") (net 29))
 (segment (start 91 94.6) (end 92 94.6) (width 0.6) (layer "B.Cu") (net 29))
 (segment (start 83.6 104.1) (end 90.9 104.1) (width 0.6) (layer "B.Cu") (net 29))
 (segment (start 93.4 94.8) (end 93.6 94.6) (width 0.6) (layer "F.Cu") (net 30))
 (segment (start 93.4 102) (end 93.4 94.8) (width 0.6) (layer "F.Cu") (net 30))
 (via (at 93.4 102) (size 0.8) (drill 0.4) (layers "F.Cu" "B.Cu") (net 30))
 (via (at 93.6 94.6) (size 0.8) (drill 0.4) (layers "F.Cu" "B.Cu") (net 30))
 (segment (start 92.96 101.56) (end 93.4 102) (width 0.6) (layer "B.Cu") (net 30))
 (segment (start 97.18 91.02) (end 97.18 54.5) (width 0.6) (layer "B.Cu") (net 30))
 (segment (start 83.6 101.56) (end 92.96 101.56) (width 0.6) (layer "B.Cu") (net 30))
 (segment (start 93.6 94.6) (end 97.18 91.02) (width 0.6) (layer "B.Cu") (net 30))
 (segment (start 98.52 96.48) (end 99 96) (width 0.6) (layer "B.Cu") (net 31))
 (segment (start 99 55.22) (end 99.72 54.5) (width 0.6) (layer "B.Cu") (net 31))
 (segment (start 99 96) (end 99 55.22) (width 0.6) (layer "B.Cu") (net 31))
 (segment (start 83.6 96.48) (end 98.52 96.48) (width 0.6) (layer "B.Cu") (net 31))
 (segment (start 107.2 64.4) (end 107.2 58.8) (width 0.6) (layer "F.Cu") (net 33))
 (via (at 107.2 58.8) (size 0.8) (drill 0.4) (layers "F.Cu" "B.Cu") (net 33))
 (via (at 107.2 64.4) (size 0.8) (drill 0.4) (layers "F.Cu" "B.Cu") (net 33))
 (segment (start 99.3475 116.84) (end 99.6 116.5875) (width 0.6) (layer "B.Cu") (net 33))
 (segment (start 99.6 105.6) (end 106.2 105.6) (width 0.6) (layer "B.Cu") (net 33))
 (segment (start 104.8 58.6) (end 104.8 54.5) (width 0.6) (layer "B.Cu") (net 33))
 (segment (start 106.6 105.2) (end 106.6 65) (width 0.6) (layer "B.Cu") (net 33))
 (segment (start 106.6 65) (end 107.2 64.4) (width 0.6) (layer "B.Cu") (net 33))
 (segment (start 99.6 116.5875) (end 99.6 105.6) (width 0.6) (layer "B.Cu") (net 33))
 (segment (start 106.2 105.6) (end 106.6 105.2) (width 0.6) (layer "B.Cu") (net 33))
 (segment (start 105 58.8) (end 104.8 58.6) (width 0.6) (layer "B.Cu") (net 33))
 (segment (start 107.2 58.8) (end 105 58.8) (width 0.6) (layer "B.Cu") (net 33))
 (segment (start 120.6 52) (end 120.6 62) (width 0.6) (layer "B.Cu") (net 36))
 (segment (start 120.4 62.2) (end 105 62.2) (width 0.6) (layer "B.Cu") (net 36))
 (segment (start 112.42 52.38) (end 112.8 52) (width 0.6) (layer "B.Cu") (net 36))
 (segment (start 112.42 54.5) (end 112.42 52.38) (width 0.6) (layer "B.Cu") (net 36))
 (segment (start 112.8 52) (end 120.6 52) (width 0.6) (layer "B.Cu") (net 36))
 (segment (start 120.6 62) (end 120.4 62.2) (width 0.6) (layer "B.Cu") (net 36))
 (segment (start 97.569499 104.030501) (end 97.569499 116.078001) (width 0.6) (layer "B.Cu") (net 36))
 (segment (start 98.2 103.4) (end 97.569499 104.030501) (width 0.6) (layer "B.Cu") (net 36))
 (segment (start 105 62.2) (end 105 102.6) (width 0.6) (layer "B.Cu") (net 36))
 (segment (start 97.569499 116.078001) (end 96.8075 116.84) (width 0.6) (layer "B.Cu") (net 36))
 (segment (start 105 102.6) (end 104.2 103.4) (width 0.6) (layer "B.Cu") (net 36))
 (segment (start 104.2 103.4) (end 98.2 103.4) (width 0.6) (layer "B.Cu") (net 36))
 (segment (start 100.38 99.02) (end 83.6 99.02) (width 0.6) (layer "B.Cu") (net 37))
 (segment (start 114.46 60.74) (end 101.86 60.74) (width 0.6) (layer "B.Cu") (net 37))
 (segment (start 114.96 54.5) (end 114.96 60.24) (width 0.6) (layer "B.Cu") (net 37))
 (segment (start 100.8 61.8) (end 100.8 98.6) (width 0.6) (layer "B.Cu") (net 37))
 (segment (start 101.86 60.74) (end 100.8 61.8) (width 0.6) (layer "B.Cu") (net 37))
 (segment (start 114.96 60.24) (end 114.46 60.74) (width 0.6) (layer "B.Cu") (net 37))
 (segment (start 100.8 98.6) (end 100.38 99.02) (width 0.6) (layer "B.Cu") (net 37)))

